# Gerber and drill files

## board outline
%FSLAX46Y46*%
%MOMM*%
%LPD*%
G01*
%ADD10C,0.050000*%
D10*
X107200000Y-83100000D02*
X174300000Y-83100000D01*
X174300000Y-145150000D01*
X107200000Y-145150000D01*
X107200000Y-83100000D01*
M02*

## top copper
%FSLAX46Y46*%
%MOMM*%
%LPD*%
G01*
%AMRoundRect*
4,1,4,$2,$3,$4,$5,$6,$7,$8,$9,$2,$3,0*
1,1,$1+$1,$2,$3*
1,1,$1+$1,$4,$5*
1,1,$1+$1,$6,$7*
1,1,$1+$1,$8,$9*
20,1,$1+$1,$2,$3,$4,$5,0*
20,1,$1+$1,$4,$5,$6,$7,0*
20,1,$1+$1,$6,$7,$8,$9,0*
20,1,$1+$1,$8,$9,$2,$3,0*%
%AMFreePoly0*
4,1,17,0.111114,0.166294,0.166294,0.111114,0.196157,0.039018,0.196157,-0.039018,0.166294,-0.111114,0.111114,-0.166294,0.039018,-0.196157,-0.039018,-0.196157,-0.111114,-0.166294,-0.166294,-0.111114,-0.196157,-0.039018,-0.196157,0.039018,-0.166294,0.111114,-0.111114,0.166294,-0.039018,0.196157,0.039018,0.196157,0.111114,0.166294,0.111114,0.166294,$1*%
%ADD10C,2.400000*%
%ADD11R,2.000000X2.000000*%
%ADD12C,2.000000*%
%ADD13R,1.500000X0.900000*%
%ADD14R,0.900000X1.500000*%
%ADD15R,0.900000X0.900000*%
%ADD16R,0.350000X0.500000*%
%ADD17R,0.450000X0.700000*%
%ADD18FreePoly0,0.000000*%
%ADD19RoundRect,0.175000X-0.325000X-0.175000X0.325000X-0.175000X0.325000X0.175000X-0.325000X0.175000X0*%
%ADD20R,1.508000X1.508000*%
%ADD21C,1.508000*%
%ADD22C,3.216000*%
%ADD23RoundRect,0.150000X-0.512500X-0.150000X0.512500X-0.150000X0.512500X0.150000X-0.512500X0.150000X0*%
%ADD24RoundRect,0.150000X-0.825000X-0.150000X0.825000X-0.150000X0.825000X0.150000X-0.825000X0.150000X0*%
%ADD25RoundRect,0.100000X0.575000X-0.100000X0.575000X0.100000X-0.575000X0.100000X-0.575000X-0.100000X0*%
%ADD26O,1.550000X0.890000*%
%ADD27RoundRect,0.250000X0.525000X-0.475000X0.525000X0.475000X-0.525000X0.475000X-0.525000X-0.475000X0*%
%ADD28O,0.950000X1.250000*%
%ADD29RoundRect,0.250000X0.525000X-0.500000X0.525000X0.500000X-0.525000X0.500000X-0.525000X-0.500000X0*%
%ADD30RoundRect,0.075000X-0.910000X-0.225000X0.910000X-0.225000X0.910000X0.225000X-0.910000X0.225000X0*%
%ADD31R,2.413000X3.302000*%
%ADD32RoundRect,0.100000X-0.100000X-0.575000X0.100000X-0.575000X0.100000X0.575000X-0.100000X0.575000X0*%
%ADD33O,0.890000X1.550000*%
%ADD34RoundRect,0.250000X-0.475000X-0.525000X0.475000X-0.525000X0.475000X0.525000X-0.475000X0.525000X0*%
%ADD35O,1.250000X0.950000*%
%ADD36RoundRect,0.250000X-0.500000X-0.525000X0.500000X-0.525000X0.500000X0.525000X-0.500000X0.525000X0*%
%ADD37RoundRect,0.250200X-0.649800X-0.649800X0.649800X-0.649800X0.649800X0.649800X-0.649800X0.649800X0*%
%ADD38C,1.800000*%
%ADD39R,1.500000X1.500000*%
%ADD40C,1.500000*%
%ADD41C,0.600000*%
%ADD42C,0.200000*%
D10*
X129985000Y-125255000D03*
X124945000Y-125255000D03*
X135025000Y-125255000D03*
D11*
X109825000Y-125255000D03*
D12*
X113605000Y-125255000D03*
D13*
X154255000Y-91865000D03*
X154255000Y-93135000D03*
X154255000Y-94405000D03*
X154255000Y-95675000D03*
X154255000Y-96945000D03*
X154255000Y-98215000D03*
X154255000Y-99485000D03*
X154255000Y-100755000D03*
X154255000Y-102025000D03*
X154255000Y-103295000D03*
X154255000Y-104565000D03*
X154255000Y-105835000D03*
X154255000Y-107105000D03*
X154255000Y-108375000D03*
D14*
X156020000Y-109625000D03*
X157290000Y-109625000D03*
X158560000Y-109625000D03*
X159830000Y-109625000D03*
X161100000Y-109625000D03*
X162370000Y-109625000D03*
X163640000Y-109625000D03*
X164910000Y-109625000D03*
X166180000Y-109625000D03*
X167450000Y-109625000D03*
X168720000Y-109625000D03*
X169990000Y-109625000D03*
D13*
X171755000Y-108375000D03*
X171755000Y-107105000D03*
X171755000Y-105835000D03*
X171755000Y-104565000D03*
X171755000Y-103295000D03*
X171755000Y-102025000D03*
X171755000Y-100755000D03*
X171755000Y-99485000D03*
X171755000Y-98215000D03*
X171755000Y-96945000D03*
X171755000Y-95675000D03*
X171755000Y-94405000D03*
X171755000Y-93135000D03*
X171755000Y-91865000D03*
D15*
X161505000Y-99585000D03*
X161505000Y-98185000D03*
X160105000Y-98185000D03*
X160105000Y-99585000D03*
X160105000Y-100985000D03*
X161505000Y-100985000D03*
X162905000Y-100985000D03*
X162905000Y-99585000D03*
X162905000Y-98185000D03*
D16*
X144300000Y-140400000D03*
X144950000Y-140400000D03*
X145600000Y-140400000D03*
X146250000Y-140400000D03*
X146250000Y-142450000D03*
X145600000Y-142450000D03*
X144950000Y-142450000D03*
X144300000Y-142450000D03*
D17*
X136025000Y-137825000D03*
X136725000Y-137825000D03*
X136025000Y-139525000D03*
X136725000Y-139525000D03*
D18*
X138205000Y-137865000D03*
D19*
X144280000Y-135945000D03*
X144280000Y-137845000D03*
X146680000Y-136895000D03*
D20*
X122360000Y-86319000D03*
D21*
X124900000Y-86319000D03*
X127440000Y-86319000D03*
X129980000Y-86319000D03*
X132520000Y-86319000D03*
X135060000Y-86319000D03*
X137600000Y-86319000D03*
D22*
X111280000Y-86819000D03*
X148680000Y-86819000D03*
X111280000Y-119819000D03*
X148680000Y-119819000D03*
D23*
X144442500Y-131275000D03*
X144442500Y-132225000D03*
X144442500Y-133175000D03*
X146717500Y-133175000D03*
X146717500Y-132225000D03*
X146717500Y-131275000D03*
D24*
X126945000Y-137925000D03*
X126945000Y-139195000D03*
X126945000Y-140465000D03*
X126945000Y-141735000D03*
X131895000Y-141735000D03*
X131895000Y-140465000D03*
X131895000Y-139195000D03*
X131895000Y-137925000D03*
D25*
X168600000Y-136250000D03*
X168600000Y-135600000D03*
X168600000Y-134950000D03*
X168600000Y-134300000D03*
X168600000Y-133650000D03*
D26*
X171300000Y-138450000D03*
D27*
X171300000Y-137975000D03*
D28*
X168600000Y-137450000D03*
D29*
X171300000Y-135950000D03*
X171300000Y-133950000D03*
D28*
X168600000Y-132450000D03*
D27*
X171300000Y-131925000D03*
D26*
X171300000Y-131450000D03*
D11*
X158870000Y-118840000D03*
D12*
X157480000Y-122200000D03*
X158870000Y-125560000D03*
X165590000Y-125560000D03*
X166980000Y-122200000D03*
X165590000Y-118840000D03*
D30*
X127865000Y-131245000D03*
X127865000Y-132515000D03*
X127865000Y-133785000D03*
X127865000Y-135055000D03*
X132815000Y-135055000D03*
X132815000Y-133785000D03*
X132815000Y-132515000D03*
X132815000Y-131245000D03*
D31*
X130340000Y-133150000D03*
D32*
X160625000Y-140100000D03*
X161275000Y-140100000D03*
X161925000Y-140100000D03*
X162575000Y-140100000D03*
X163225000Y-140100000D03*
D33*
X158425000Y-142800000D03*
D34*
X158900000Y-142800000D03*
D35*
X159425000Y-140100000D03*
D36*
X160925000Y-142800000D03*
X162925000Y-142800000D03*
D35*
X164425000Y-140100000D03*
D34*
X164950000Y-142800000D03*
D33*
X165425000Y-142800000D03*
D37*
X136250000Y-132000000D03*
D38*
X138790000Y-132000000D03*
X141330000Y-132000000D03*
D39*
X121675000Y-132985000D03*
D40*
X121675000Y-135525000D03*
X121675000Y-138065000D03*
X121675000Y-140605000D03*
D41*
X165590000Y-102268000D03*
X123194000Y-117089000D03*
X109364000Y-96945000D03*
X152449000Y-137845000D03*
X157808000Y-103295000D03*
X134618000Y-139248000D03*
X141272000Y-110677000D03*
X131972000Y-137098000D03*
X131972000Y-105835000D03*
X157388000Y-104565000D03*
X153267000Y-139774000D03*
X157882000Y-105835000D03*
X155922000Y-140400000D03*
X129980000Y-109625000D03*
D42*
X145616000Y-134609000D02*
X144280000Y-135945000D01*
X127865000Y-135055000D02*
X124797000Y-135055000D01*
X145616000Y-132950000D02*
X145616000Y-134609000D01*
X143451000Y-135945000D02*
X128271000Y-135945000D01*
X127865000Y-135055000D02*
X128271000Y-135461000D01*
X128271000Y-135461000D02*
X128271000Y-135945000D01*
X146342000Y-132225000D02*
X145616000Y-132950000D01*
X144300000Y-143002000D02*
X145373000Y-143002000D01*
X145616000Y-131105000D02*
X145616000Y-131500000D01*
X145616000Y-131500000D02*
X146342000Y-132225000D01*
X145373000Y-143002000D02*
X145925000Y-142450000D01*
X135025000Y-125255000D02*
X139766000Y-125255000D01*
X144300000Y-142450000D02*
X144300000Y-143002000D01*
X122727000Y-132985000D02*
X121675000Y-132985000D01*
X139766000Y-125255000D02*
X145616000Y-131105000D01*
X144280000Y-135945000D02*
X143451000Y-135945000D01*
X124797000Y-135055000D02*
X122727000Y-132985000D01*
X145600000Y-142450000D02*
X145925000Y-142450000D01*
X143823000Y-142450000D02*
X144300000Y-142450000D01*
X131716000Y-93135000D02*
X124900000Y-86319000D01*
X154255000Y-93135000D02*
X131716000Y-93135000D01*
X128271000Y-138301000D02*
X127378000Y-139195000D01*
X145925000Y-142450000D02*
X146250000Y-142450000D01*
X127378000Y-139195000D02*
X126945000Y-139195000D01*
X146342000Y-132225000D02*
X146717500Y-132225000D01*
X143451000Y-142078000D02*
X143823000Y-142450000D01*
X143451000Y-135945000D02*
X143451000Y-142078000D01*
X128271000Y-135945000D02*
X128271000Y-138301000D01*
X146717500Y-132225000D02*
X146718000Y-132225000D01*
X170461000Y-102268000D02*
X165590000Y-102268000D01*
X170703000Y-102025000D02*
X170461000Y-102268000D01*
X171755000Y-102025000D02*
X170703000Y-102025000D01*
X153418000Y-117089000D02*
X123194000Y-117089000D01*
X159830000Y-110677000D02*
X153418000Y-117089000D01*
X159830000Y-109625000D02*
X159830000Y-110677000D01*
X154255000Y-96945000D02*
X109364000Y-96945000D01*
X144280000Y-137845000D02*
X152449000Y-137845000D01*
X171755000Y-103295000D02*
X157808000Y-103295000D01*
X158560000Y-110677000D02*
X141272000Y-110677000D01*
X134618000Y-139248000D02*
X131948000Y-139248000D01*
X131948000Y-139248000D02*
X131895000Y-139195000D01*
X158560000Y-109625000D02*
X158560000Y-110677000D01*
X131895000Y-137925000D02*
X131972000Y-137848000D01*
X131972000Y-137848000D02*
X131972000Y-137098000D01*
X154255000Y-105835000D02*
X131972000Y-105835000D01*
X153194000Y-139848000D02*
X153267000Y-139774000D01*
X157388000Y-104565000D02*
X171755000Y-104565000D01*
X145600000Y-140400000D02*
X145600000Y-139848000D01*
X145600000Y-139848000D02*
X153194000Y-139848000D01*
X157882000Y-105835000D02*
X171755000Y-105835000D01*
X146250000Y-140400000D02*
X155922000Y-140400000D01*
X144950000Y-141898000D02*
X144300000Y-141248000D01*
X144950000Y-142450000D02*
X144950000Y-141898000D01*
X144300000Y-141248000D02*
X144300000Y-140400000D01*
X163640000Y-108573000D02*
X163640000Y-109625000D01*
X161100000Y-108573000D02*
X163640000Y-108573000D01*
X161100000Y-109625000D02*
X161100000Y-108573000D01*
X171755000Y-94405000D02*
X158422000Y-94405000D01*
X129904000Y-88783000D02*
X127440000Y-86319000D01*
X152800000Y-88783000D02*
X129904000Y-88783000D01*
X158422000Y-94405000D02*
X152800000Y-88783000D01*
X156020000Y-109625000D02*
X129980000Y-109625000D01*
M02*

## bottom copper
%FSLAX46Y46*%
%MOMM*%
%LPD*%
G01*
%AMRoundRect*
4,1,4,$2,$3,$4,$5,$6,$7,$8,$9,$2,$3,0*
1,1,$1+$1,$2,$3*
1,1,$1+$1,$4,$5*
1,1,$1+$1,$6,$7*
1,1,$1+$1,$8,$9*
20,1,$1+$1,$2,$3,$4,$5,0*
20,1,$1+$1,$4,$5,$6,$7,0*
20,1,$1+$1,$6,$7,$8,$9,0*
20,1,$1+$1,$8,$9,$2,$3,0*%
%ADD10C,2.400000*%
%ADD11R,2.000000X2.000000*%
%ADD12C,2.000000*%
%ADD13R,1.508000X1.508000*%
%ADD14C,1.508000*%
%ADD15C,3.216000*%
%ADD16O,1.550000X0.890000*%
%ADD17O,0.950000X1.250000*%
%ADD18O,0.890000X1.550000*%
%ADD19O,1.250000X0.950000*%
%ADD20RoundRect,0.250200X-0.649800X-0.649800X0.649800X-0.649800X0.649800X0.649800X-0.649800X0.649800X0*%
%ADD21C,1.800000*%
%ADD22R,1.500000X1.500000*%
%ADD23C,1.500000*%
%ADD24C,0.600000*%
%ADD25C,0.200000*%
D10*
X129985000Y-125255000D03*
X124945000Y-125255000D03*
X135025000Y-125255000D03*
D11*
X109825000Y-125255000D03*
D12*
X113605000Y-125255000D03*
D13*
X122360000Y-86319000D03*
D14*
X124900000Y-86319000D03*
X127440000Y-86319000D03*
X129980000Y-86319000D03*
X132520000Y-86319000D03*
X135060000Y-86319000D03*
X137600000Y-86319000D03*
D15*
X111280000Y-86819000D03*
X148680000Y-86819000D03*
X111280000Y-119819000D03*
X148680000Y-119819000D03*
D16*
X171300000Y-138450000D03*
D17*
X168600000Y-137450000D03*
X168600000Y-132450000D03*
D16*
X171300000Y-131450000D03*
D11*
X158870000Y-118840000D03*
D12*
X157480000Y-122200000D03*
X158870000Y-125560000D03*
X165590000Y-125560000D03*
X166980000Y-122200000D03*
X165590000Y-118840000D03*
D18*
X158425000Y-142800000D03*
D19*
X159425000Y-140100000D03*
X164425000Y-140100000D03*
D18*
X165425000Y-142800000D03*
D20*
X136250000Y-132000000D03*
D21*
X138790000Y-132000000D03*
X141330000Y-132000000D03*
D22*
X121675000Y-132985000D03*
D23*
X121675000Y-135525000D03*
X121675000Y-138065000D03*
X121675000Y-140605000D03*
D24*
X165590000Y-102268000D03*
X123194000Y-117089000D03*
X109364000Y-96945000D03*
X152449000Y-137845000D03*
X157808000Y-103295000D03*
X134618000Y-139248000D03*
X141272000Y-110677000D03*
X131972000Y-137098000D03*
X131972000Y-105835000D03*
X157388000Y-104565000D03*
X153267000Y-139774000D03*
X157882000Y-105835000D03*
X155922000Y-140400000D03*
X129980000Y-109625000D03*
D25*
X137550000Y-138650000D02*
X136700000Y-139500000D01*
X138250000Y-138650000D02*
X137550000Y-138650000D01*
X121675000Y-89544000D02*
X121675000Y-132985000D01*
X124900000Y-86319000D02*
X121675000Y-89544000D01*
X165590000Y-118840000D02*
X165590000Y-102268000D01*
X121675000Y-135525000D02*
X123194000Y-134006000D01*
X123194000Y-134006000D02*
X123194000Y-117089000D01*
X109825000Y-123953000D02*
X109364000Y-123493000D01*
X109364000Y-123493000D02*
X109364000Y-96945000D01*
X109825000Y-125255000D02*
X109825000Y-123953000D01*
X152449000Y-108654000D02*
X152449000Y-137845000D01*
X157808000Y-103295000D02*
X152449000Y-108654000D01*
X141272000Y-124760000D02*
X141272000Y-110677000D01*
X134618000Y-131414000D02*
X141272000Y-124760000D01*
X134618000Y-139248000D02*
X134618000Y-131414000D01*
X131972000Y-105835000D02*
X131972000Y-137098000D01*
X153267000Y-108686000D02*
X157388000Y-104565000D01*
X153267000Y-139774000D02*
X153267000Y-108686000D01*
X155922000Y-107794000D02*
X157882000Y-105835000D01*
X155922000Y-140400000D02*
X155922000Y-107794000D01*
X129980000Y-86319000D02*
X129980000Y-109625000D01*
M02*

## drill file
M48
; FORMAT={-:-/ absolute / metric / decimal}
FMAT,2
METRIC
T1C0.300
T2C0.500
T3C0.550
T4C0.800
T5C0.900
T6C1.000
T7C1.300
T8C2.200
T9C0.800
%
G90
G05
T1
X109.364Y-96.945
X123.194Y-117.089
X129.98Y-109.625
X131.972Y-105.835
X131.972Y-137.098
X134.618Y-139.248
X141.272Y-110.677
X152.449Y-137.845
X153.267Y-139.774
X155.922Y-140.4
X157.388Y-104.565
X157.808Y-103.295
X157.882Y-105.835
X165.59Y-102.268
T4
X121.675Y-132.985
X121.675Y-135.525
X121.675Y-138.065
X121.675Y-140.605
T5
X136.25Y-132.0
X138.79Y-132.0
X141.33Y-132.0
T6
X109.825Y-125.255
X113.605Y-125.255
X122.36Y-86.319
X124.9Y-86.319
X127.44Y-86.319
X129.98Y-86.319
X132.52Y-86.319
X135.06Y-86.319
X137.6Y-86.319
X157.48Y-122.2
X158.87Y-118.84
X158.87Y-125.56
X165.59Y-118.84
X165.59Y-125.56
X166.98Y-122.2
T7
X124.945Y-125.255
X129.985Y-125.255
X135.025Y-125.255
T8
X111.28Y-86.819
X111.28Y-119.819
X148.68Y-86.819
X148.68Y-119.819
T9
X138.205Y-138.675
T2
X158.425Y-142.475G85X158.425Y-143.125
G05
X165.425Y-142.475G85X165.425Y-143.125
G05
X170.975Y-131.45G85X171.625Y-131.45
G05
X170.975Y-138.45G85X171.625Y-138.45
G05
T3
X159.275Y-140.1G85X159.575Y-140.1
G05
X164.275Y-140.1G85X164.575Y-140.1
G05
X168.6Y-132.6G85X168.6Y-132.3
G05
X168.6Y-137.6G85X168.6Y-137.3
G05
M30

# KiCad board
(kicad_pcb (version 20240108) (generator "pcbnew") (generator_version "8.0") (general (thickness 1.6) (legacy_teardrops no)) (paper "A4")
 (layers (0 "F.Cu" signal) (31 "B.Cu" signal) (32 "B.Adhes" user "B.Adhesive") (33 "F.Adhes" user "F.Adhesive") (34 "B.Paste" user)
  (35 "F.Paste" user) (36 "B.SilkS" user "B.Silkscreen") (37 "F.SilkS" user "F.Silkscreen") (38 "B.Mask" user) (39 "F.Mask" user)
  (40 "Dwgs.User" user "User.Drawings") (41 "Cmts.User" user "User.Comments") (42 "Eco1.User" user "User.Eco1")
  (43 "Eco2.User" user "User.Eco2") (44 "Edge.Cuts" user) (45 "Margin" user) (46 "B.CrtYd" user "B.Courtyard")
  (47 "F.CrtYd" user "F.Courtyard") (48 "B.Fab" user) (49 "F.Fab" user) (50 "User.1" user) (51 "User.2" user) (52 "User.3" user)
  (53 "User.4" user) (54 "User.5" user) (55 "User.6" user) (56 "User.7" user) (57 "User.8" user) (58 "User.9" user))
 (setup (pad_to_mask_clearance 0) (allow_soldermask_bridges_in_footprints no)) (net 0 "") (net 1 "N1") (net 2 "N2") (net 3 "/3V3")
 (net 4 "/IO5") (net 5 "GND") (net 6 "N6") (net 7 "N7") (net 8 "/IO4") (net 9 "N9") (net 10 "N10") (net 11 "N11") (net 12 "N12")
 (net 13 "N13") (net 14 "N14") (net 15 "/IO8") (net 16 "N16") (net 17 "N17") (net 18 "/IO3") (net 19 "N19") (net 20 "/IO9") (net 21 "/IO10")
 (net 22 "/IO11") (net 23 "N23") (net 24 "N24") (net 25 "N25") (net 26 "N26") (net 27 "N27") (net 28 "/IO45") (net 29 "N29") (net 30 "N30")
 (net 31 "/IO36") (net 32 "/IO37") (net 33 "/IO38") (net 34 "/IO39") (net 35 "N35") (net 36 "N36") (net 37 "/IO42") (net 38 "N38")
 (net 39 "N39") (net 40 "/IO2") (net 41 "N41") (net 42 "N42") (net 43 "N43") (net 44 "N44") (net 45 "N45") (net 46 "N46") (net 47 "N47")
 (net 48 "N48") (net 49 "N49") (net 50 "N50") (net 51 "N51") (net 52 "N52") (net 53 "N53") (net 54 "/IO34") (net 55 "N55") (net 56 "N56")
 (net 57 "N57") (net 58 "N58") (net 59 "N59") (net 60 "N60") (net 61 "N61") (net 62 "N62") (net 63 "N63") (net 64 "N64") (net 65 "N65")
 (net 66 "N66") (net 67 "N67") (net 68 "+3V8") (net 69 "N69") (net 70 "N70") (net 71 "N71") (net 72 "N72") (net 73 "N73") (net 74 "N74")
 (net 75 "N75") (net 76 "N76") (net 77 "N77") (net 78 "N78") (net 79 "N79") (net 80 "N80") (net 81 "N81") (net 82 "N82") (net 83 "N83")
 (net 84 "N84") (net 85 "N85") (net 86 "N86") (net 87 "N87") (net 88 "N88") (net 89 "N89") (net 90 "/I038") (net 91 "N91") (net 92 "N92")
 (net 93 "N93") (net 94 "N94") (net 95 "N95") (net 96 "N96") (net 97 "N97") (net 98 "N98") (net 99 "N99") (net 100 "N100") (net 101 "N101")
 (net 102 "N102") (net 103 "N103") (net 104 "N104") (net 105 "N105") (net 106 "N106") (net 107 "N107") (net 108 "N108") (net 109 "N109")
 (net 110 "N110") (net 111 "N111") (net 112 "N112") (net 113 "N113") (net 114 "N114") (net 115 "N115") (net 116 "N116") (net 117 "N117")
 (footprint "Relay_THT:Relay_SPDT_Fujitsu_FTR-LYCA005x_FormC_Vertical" (layer "F.Cu") (at 109.825 125.255)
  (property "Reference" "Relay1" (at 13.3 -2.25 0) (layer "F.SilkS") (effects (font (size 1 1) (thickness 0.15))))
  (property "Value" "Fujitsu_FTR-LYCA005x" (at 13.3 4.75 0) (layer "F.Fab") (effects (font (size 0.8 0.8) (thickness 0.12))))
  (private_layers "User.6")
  (pad "11" thru_hole circle (at 20.16 0) (size 2.4 2.4) (drill 1.3) (layers "*.Cu" "*.Mask") (remove_unused_layers no) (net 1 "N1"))
  (pad "12" thru_hole circle (at 15.12 0) (size 2.4 2.4) (drill 1.3) (layers "*.Cu" "*.Mask") (remove_unused_layers no) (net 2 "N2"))
  (pad "14" thru_hole circle (at 25.2 0) (size 2.4 2.4) (drill 1.3) (layers "*.Cu" "*.Mask") (remove_unused_layers no) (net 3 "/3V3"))
  (pad "A1" thru_hole rect (at 0 0) (size 2 2) (drill 1) (layers "*.Cu" "*.Mask") (remove_unused_layers no) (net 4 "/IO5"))
  (pad "A2" thru_hole circle (at 3.78 0) (size 2 2) (drill 1) (layers "*.Cu" "*.Mask") (remove_unused_layers no) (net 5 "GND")))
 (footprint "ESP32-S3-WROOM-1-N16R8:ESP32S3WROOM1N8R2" (layer "F.Cu") (at 163.005 97.125)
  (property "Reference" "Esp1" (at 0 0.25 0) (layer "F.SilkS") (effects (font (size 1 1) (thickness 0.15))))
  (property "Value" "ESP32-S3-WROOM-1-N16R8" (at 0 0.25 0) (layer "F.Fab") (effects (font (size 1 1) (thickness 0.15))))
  (pad "1" smd rect (at -8.75 -5.26) (size 1.5 0.9) (layers "F.Cu" "F.Paste" "F.Mask") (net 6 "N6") (solder_mask_margin 0.102))
  (pad "2" smd rect (at -8.75 -3.99) (size 1.5 0.9) (layers "F.Cu" "F.Paste" "F.Mask") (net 3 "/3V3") (solder_mask_margin 0.102))
  (pad "3" smd rect (at -8.75 -2.72) (size 1.5 0.9) (layers "F.Cu" "F.Paste" "F.Mask") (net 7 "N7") (solder_mask_margin 0.102))
  (pad "4" smd rect (at -8.75 -1.45) (size 1.5 0.9) (layers "F.Cu" "F.Paste" "F.Mask") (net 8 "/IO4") (solder_mask_margin 0.102))
  (pad "5" smd rect (at -8.75 -0.18) (size 1.5 0.9) (layers "F.Cu" "F.Paste" "F.Mask") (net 4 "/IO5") (solder_mask_margin 0.102))
  (pad "6" smd rect (at -8.75 1.09) (size 1.5 0.9) (layers "F.Cu" "F.Paste" "F.Mask") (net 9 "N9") (solder_mask_margin 0.102))
  (pad "7" smd rect (at -8.75 2.36) (size 1.5 0.9) (layers "F.Cu" "F.Paste" "F.Mask") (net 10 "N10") (solder_mask_margin 0.102))
  (pad "8" smd rect (at -8.75 3.63) (size 1.5 0.9) (layers "F.Cu" "F.Paste" "F.Mask") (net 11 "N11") (solder_mask_margin 0.102))
  (pad "9" smd rect (at -8.75 4.9) (size 1.5 0.9) (layers "F.Cu" "F.Paste" "F.Mask") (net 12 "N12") (solder_mask_margin 0.102))
  (pad "10" smd rect (at -8.75 6.17) (size 1.5 0.9) (layers "F.Cu" "F.Paste" "F.Mask") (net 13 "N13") (solder_mask_margin 0.102))
  (pad "11" smd rect (at -8.75 7.44) (size 1.5 0.9) (layers "F.Cu" "F.Paste" "F.Mask") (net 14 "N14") (solder_mask_margin 0.102))
  (pad "12" smd rect (at -8.75 8.71) (size 1.5 0.9) (layers "F.Cu" "F.Paste" "F.Mask") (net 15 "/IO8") (solder_mask_margin 0.102))
  (pad "13" smd rect (at -8.75 9.98) (size 1.5 0.9) (layers "F.Cu" "F.Paste" "F.Mask") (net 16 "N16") (solder_mask_margin 0.102))
  (pad "14" smd rect (at -8.75 11.25) (size 1.5 0.9) (layers "F.Cu" "F.Paste" "F.Mask") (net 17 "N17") (solder_mask_margin 0.102))
  (pad "15" smd rect (at -6.985 12.5) (size 0.9 1.5) (layers "F.Cu" "F.Paste" "F.Mask") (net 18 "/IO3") (solder_mask_margin 0.102))
  (pad "16" smd rect (at -5.715 12.5) (size 0.9 1.5) (layers "F.Cu" "F.Paste" "F.Mask") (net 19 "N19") (solder_mask_margin 0.102))
  (pad "17" smd rect (at -4.445 12.5) (size 0.9 1.5) (layers "F.Cu" "F.Paste" "F.Mask") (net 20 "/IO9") (solder_mask_margin 0.102))
  (pad "18" smd rect (at -3.175 12.5) (size 0.9 1.5) (layers "F.Cu" "F.Paste" "F.Mask") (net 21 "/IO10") (solder_mask_margin 0.102))
  (pad "19" smd rect (at -1.905 12.5) (size 0.9 1.5) (layers "F.Cu" "F.Paste" "F.Mask") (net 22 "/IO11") (solder_mask_margin 0.102))
  (pad "20" smd rect (at -0.635 12.5) (size 0.9 1.5) (layers "F.Cu" "F.Paste" "F.Mask") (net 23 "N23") (solder_mask_margin 0.102))
  (pad "21" smd rect (at 0.635 12.5) (size 0.9 1.5) (layers "F.Cu" "F.Paste" "F.Mask") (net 22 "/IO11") (solder_mask_margin 0.102))
  (pad "22" smd rect (at 1.905 12.5) (size 0.9 1.5) (layers "F.Cu" "F.Paste" "F.Mask") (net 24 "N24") (solder_mask_margin 0.102))
  (pad "23" smd rect (at 3.175 12.5) (size 0.9 1.5) (layers "F.Cu" "F.Paste" "F.Mask") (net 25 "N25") (solder_mask_margin 0.102))
  (pad "24" smd rect (at 4.445 12.5) (size 0.9 1.5) (layers "F.Cu" "F.Paste" "F.Mask") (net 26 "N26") (solder_mask_margin 0.102))
  (pad "25" smd rect (at 5.715 12.5) (size 0.9 1.5) (layers "F.Cu" "F.Paste" "F.Mask") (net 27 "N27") (solder_mask_margin 0.102))
  (pad "26" smd rect (at 6.985 12.5) (size 0.9 1.5) (layers "F.Cu" "F.Paste" "F.Mask") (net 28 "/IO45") (solder_mask_margin 0.102))
  (pad "27" smd rect (at 8.75 11.25) (size 1.5 0.9) (layers "F.Cu" "F.Paste" "F.Mask") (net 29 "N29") (solder_mask_margin 0.102))
  (pad "28" smd rect (at 8.75 9.98) (size 1.5 0.9) (layers "F.Cu" "F.Paste" "F.Mask") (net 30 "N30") (solder_mask_margin 0.102))
  (pad "29" smd rect (at 8.75 8.71) (size 1.5 0.9) (layers "F.Cu" "F.Paste" "F.Mask") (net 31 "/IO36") (solder_mask_margin 0.102))
  (pad "30" smd rect (at 8.75 7.44) (size 1.5 0.9) (layers "F.Cu" "F.Paste" "F.Mask") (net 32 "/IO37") (solder_mask_margin 0.102))
  (pad "31" smd rect (at 8.75 6.17) (size 1.5 0.9) (layers "F.Cu" "F.Paste" "F.Mask") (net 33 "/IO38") (solder_mask_margin 0.102))
  (pad "32" smd rect (at 8.75 4.9) (size 1.5 0.9) (layers "F.Cu" "F.Paste" "F.Mask") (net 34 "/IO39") (solder_mask_margin 0.102))
  (pad "33" smd rect (at 8.75 3.63) (size 1.5 0.9) (layers "F.Cu" "F.Paste" "F.Mask") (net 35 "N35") (solder_mask_margin 0.102))
  (pad "34" smd rect (at 8.75 2.36) (size 1.5 0.9) (layers "F.Cu" "F.Paste" "F.Mask") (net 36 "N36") (solder_mask_margin 0.102))
  (pad "35" smd rect (at 8.75 1.09) (size 1.5 0.9) (layers "F.Cu" "F.Paste" "F.Mask") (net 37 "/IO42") (solder_mask_margin 0.102))
  (pad "36" smd rect (at 8.75 -0.18) (size 1.5 0.9) (layers "F.Cu" "F.Paste" "F.Mask") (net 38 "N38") (solder_mask_margin 0.102))
  (pad "37" smd rect (at 8.75 -1.45) (size 1.5 0.9) (layers "F.Cu" "F.Paste" "F.Mask") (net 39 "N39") (solder_mask_margin 0.102))
  (pad "38" smd rect (at 8.75 -2.72) (size 1.5 0.9) (layers "F.Cu" "F.Paste" "F.Mask") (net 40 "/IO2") (solder_mask_margin 0.102))
  (pad "39" smd rect (at 8.75 -3.99) (size 1.5 0.9) (layers "F.Cu" "F.Paste" "F.Mask") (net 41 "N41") (solder_mask_margin 0.102))
  (pad "40" smd rect (at 8.75 -5.26) (size 1.5 0.9) (layers "F.Cu" "F.Paste" "F.Mask") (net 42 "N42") (solder_mask_margin 0.102))
  (pad "41" smd rect (at -1.5 2.46) (size 0.9 0.9) (layers "F.Cu" "F.Paste" "F.Mask") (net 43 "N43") (solder_mask_margin 0.102))
  (pad "42" smd rect (at -1.5 1.06) (size 0.9 0.9) (layers "F.Cu" "F.Paste" "F.Mask") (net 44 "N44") (solder_mask_margin 0.102))
  (pad "43" smd rect (at -2.9 1.06) (size 0.9 0.9) (layers "F.Cu" "F.Paste" "F.Mask") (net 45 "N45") (solder_mask_margin 0.102))
  (pad "44" smd rect (at -2.9 2.46) (size 0.9 0.9) (layers "F.Cu" "F.Paste" "F.Mask") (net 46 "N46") (solder_mask_margin 0.102))
  (pad "45" smd rect (at -2.9 3.86) (size 0.9 0.9) (layers "F.Cu" "F.Paste" "F.Mask") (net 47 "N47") (solder_mask_margin 0.102))
  (pad "46" smd rect (at -1.5 3.86) (size 0.9 0.9) (layers "F.Cu" "F.Paste" "F.Mask") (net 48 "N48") (solder_mask_margin 0.102))
  (pad "47" smd rect (at -0.1 3.86) (size 0.9 0.9) (layers "F.Cu" "F.Paste" "F.Mask") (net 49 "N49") (solder_mask_margin 0.102))
  (pad "48" smd rect (at -0.1 2.46) (size 0.9 0.9) (layers "F.Cu" "F.Paste" "F.Mask") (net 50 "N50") (solder_mask_margin 0.102))
  (pad "49" smd rect (at -0.1 1.06) (size 0.9 0.9) (layers "F.Cu" "F.Paste" "F.Mask") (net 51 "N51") (solder_mask_margin 0.102)))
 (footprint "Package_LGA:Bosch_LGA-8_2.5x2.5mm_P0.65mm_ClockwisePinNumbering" (layer "F.Cu") (at 145.275 141.425)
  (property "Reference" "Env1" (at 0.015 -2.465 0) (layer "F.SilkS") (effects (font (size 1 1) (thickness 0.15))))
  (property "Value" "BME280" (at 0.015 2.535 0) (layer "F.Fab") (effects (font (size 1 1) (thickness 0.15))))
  (pad "1" smd rect (at -0.975 -1.025 90) (size 0.5 0.35) (layers "F.Cu" "F.Paste" "F.Mask") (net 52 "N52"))
  (pad "2" smd rect (at -0.325 -1.025 90) (size 0.5 0.35) (layers "F.Cu" "F.Paste" "F.Mask") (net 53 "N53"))
  (pad "3" smd rect (at 0.325 -1.025 90) (size 0.5 0.35) (layers "F.Cu" "F.Paste" "F.Mask") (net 32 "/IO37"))
  (pad "4" smd rect (at 0.975 -1.025 90) (size 0.5 0.35) (layers "F.Cu" "F.Paste" "F.Mask") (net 31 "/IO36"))
  (pad "5" smd rect (at 0.975 1.025 90) (size 0.5 0.35) (layers "F.Cu" "F.Paste" "F.Mask") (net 3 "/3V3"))
  (pad "6" smd rect (at 0.325 1.025 90) (size 0.5 0.35) (layers "F.Cu" "F.Paste" "F.Mask") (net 3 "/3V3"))
  (pad "7" smd rect (at -0.325 1.025 90) (size 0.5 0.35) (layers "F.Cu" "F.Paste" "F.Mask") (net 52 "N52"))
  (pad "8" smd rect (at -0.975 1.025 90) (size 0.5 0.35) (layers "F.Cu" "F.Paste" "F.Mask") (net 3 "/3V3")))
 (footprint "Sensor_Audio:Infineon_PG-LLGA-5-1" (layer "F.Cu") (at 137.525 138.675)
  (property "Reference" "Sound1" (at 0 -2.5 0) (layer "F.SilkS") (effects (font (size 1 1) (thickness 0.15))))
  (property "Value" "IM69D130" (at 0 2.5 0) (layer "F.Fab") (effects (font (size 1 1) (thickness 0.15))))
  (pad "" smd custom (at -1.5 -0.725) (size 0.3 0.3) (layers "F.Paste") (zone_connect 0) (options (clearance outline) (anchor circle))
   (primitives))
  (pad "" smd custom (at -1.5 0.725) (size 0.3 0.3) (layers "F.Paste") (zone_connect 0) (options (clearance outline) (anchor circle))
   (primitives))
  (pad "" smd custom (at -0.8 -0.725) (size 0.3 0.3) (layers "F.Paste") (zone_connect 0) (options (clearance outline) (anchor circle))
   (primitives))
  (pad "" smd custom (at -0.8 0.725) (size 0.3 0.3) (layers "F.Paste") (zone_connect 0) (options (clearance outline) (anchor circle))
   (primitives))
  (pad "" smd custom (at -0.12 0) (size 0.3 0.3) (layers "F.Paste") (zone_connect 0) (options (clearance outline) (anchor circle))
   (primitives))
  (pad "" smd custom (at 0.28 -0.693) (size 0.3 0.3) (layers "F.Paste") (zone_connect 0) (options (clearance outline) (anchor circle))
   (primitives))
  (pad "" smd custom (at 0.28 0.693) (size 0.3 0.3) (layers "F.Paste") (zone_connect 0) (options (clearance outline) (anchor circle))
   (primitives))
  (pad "" np_thru_hole circle (at 0.68 0) (size 0.8 0.8) (drill 0.8) (layers "*.Cu" "*.Mask"))
  (pad "" smd custom (at 1.08 -0.693) (size 0.3 0.3) (layers "F.Paste") (zone_connect 0) (options (clearance outline) (anchor circle))
   (primitives))
  (pad "" smd custom (at 1.08 0.693) (size 0.3 0.3) (layers "F.Paste") (zone_connect 0) (options (clearance outline) (anchor circle))
   (primitives))
  (pad "" smd custom (at 1.48 0) (size 0.3 0.3) (layers "F.Paste") (zone_connect 0) (options (clearance outline) (anchor circle))
   (primitives))
  (pad "1" smd rect (at -1.5 -0.85) (size 0.45 0.7) (layers "F.Cu" "F.Mask") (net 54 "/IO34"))
  (pad "2" smd rect (at -0.8 -0.85) (size 0.45 0.7) (layers "F.Cu" "F.Mask") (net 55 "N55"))
  (pad "3" smd rect (at -1.5 0.85) (size 0.45 0.7) (layers "F.Cu" "F.Mask") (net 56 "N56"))
  (pad "4" smd rect (at -0.8 0.85) (size 0.45 0.7) (layers "F.Cu" "F.Mask") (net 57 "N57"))
  (pad "5" smd custom (at 0.68 -0.81) (size 0.4 0.4) (layers "F.Cu" "F.Mask") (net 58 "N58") (zone_connect 0)
   (options (clearance outline) (anchor circle)) (primitives)))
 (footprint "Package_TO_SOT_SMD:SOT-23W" (layer "F.Cu") (at 145.48 136.895)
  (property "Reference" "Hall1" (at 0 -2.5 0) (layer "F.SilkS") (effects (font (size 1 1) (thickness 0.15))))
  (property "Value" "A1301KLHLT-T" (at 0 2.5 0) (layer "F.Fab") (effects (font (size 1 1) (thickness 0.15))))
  (pad "1" smd roundrect (at -1.2 -0.95) (size 1 0.7) (layers "F.Cu" "F.Paste" "F.Mask") (roundrect_rratio 0.25) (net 3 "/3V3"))
  (pad "2" smd roundrect (at -1.2 0.95) (size 1 0.7) (layers "F.Cu" "F.Paste" "F.Mask") (roundrect_rratio 0.25) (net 33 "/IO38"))
  (pad "3" smd roundrect (at 1.2 0) (size 1 0.7) (layers "F.Cu" "F.Paste" "F.Mask") (roundrect_rratio 0.25) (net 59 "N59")))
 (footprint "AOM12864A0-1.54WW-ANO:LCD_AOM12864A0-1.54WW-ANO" (layer "F.Cu") (at 129.98 103.319)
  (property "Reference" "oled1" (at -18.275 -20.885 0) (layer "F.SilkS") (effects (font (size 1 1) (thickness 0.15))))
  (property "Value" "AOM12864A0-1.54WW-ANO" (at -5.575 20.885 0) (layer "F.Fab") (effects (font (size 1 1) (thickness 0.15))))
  (pad "1" thru_hole rect (at -7.62 -17) (size 1.508 1.508) (drill 1) (layers "*.Cu" "*.Mask") (remove_unused_layers no) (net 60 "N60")
   (solder_mask_margin 0.102))
  (pad "2" thru_hole circle (at -5.08 -17) (size 1.508 1.508) (drill 1) (layers "*.Cu" "*.Mask") (remove_unused_layers no) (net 3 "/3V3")
   (solder_mask_margin 0.102))
  (pad "3" thru_hole circle (at -2.54 -17) (size 1.508 1.508) (drill 1) (layers "*.Cu" "*.Mask") (remove_unused_layers no) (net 40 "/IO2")
   (solder_mask_margin 0.102))
  (pad "4" thru_hole circle (at 0 -17) (size 1.508 1.508) (drill 1) (layers "*.Cu" "*.Mask") (remove_unused_layers no) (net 18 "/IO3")
   (solder_mask_margin 0.102))
  (pad "5" thru_hole circle (at 2.54 -17) (size 1.508 1.508) (drill 1) (layers "*.Cu" "*.Mask") (remove_unused_layers no) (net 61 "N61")
   (solder_mask_margin 0.102))
  (pad "6" thru_hole circle (at 5.08 -17) (size 1.508 1.508) (drill 1) (layers "*.Cu" "*.Mask") (remove_unused_layers no) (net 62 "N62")
   (solder_mask_margin 0.102))
  (pad "7" thru_hole circle (at 7.62 -17) (size 1.508 1.508) (drill 1) (layers "*.Cu" "*.Mask") (remove_unused_layers no) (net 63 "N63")
   (solder_mask_margin 0.102))
  (pad "P1" thru_hole circle (at -18.7 -16.5) (size 3.216 3.216) (drill 2.2) (layers "*.Cu" "*.Mask") (remove_unused_layers no)
   (solder_mask_margin 0.102))
  (pad "P2" thru_hole circle (at 18.7 -16.5) (size 3.216 3.216) (drill 2.2) (layers "*.Cu" "*.Mask") (remove_unused_layers no)
   (solder_mask_margin 0.102))
  (pad "P3" thru_hole circle (at -18.7 16.5) (size 3.216 3.216) (drill 2.2) (layers "*.Cu" "*.Mask") (remove_unused_layers no)
   (solder_mask_margin 0.102))
  (pad "P4" thru_hole circle (at 18.7 16.5) (size 3.216 3.216) (drill 2.2) (layers "*.Cu" "*.Mask") (remove_unused_layers no)
   (solder_mask_margin 0.102)))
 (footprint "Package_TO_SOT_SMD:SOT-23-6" (layer "F.Cu") (at 145.58 132.225)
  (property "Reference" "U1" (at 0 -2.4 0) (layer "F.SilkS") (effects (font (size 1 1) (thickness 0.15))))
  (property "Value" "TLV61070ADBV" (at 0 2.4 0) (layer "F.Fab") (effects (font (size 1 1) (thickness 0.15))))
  (pad "1" smd roundrect (at -1.1375 -0.95) (size 1.325 0.6) (layers "F.Cu" "F.Paste" "F.Mask") (roundrect_rratio 0.25) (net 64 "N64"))
  (pad "2" smd roundrect (at -1.1375 0) (size 1.325 0.6) (layers "F.Cu" "F.Paste" "F.Mask") (roundrect_rratio 0.25) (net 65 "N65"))
  (pad "3" smd roundrect (at -1.1375 0.95) (size 1.325 0.6) (layers "F.Cu" "F.Paste" "F.Mask") (roundrect_rratio 0.25) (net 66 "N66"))
  (pad "4" smd roundrect (at 1.1375 0.95) (size 1.325 0.6) (layers "F.Cu" "F.Paste" "F.Mask") (roundrect_rratio 0.25) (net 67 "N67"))
  (pad "5" smd roundrect (at 1.1375 0) (size 1.325 0.6) (layers "F.Cu" "F.Paste" "F.Mask") (roundrect_rratio 0.25) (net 3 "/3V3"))
  (pad "6" smd roundrect (at 1.1375 -0.95) (size 1.325 0.6) (layers "F.Cu" "F.Paste" "F.Mask") (roundrect_rratio 0.25) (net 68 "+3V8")))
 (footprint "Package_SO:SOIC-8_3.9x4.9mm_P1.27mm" (layer "F.Cu") (at 129.42 139.83)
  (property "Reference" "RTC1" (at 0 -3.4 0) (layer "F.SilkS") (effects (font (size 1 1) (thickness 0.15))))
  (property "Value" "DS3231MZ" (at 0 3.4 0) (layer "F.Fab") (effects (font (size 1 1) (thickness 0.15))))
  (pad "1" smd roundrect (at -2.475 -1.905) (size 1.95 0.6) (layers "F.Cu" "F.Paste" "F.Mask") (roundrect_rratio 0.25) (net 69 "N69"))
  (pad "2" smd roundrect (at -2.475 -0.635) (size 1.95 0.6) (layers "F.Cu" "F.Paste" "F.Mask") (roundrect_rratio 0.25) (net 3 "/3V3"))
  (pad "3" smd roundrect (at -2.475 0.635) (size 1.95 0.6) (layers "F.Cu" "F.Paste" "F.Mask") (roundrect_rratio 0.25) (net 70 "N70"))
  (pad "4" smd roundrect (at -2.475 1.905) (size 1.95 0.6) (layers "F.Cu" "F.Paste" "F.Mask") (roundrect_rratio 0.25) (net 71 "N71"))
  (pad "5" smd roundrect (at 2.475 1.905) (size 1.95 0.6) (layers "F.Cu" "F.Paste" "F.Mask") (roundrect_rratio 0.25) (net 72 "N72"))
  (pad "6" smd roundrect (at 2.475 0.635) (size 1.95 0.6) (layers "F.Cu" "F.Paste" "F.Mask") (roundrect_rratio 0.25) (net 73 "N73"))
  (pad "7" smd roundrect (at 2.475 -0.635) (size 1.95 0.6) (layers "F.Cu" "F.Paste" "F.Mask") (roundrect_rratio 0.25) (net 20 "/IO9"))
  (pad "8" smd roundrect (at 2.475 -1.905) (size 1.95 0.6) (layers "F.Cu" "F.Paste" "F.Mask") (roundrect_rratio 0.25) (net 15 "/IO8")))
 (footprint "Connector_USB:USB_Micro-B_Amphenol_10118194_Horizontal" (layer "F.Cu") (at 170 134.95 90)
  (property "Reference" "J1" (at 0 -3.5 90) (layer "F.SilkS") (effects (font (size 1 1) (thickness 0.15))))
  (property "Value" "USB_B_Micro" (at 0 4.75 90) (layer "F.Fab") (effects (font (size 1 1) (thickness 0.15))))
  (pad "" smd oval (at -3.5 1.3 90) (size 0.89 1.55) (layers "F.Paste"))
  (pad "" smd oval (at -2.5 -1.4 90) (size 1.25 0.95) (layers "F.Paste"))
  (pad "" smd oval (at 2.5 -1.4 90) (size 1.25 0.95) (layers "F.Paste"))
  (pad "" smd oval (at 3.5 1.3 90) (size 0.89 1.55) (layers "F.Paste"))
  (pad "1" smd roundrect (at -1.3 -1.4 90) (size 0.4 1.35) (layers "F.Cu" "F.Paste" "F.Mask") (roundrect_rratio 0.25) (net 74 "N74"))
  (pad "2" smd roundrect (at -0.65 -1.4 90) (size 0.4 1.35) (layers "F.Cu" "F.Paste" "F.Mask") (roundrect_rratio 0.25) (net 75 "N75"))
  (pad "3" smd roundrect (at 0 -1.4 90) (size 0.4 1.35) (layers "F.Cu" "F.Paste" "F.Mask") (roundrect_rratio 0.25) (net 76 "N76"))
  (pad "4" smd roundrect (at 0.65 -1.4 90) (size 0.4 1.35) (layers "F.Cu" "F.Paste" "F.Mask") (roundrect_rratio 0.25) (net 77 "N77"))
  (pad "5" smd roundrect (at 1.3 -1.4 90) (size 0.4 1.35) (layers "F.Cu" "F.Paste" "F.Mask") (roundrect_rratio 0.25) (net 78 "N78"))
  (pad "6" thru_hole oval (at -3.5 1.3 90) (size 0.89 1.55) (drill oval 0.5 1.15) (layers "*.Cu" "*.Mask") (remove_unused_layers no)
   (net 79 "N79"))
  (pad "6" smd roundrect (at -3.025 1.3 90) (size 1.45 1.55) (layers "F.Cu" "F.Paste" "F.Mask") (roundrect_rratio 0.1724137931)
   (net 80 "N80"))
  (pad "6" thru_hole oval (at -2.5 -1.4 90) (size 1.25 0.95) (drill oval 0.85 0.55) (layers "*.Cu" "*.Mask") (remove_unused_layers no)
   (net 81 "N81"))
  (pad "6" smd roundrect (at -1 1.3 90) (size 1.5 1.55) (layers "F.Cu" "F.Paste" "F.Mask") (roundrect_rratio 0.1666666667) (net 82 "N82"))
  (pad "6" smd roundrect (at 1 1.3 90) (size 1.5 1.55) (layers "F.Cu" "F.Paste" "F.Mask") (roundrect_rratio 0.1666666667) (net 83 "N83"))
  (pad "6" thru_hole oval (at 2.5 -1.4 90) (size 1.25 0.95) (drill oval 0.85 0.55) (layers "*.Cu" "*.Mask") (remove_unused_layers no)
   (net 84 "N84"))
  (pad "6" smd roundrect (at 3.025 1.3 90) (size 1.45 1.55) (layers "F.Cu" "F.Paste" "F.Mask") (roundrect_rratio 0.1724137931)
   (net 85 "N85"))
  (pad "6" thru_hole oval (at 3.5 1.3 90) (size 0.89 1.55) (drill oval 0.5 1.15) (layers "*.Cu" "*.Mask") (remove_unused_layers no)
   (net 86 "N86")))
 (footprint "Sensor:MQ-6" (layer "F.Cu") (at 158.87 118.84)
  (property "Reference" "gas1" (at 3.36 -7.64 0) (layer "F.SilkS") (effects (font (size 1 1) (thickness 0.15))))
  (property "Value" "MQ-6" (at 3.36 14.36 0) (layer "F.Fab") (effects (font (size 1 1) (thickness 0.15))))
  (pad "1" thru_hole rect (at 0 0) (size 2 2) (drill 1) (layers "*.Cu" "*.Mask") (remove_unused_layers no) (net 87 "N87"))
  (pad "2" thru_hole circle (at -1.39 3.36) (size 2 2) (drill 1) (layers "*.Cu" "*.Mask") (remove_unused_layers no) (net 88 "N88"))
  (pad "3" thru_hole circle (at 0 6.72 90) (size 2 2) (drill 1) (layers "*.Cu" "*.Mask") (remove_unused_layers no) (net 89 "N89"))
  (pad "4" thru_hole circle (at 6.72 6.72 180) (size 2 2) (drill 1) (layers "*.Cu" "*.Mask") (remove_unused_layers no) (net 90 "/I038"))
  (pad "5" thru_hole circle (at 8.11 3.36) (size 2 2) (drill 1) (layers "*.Cu" "*.Mask") (remove_unused_layers no) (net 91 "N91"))
  (pad "6" thru_hole circle (at 6.72 0 270) (size 2 2) (drill 1) (layers "*.Cu" "*.Mask") (remove_unused_layers no) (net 34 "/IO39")))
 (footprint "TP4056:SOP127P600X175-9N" (layer "F.Cu") (at 130.34 133.15)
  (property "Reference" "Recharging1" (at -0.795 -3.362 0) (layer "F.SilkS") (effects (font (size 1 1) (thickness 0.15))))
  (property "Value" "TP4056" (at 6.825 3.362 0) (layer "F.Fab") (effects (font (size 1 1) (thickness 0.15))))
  (pad "1" smd roundrect (at -2.475 -1.905) (size 1.97 0.6) (layers "F.Cu" "F.Paste" "F.Mask") (roundrect_rratio 0.125) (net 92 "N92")
   (solder_mask_margin 0.102))
  (pad "2" smd roundrect (at -2.475 -0.635) (size 1.97 0.6) (layers "F.Cu" "F.Paste" "F.Mask") (roundrect_rratio 0.125) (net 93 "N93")
   (solder_mask_margin 0.102))
  (pad "3" smd roundrect (at -2.475 0.635) (size 1.97 0.6) (layers "F.Cu" "F.Paste" "F.Mask") (roundrect_rratio 0.125) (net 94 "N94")
   (solder_mask_margin 0.102))
  (pad "4" smd roundrect (at -2.475 1.905) (size 1.97 0.6) (layers "F.Cu" "F.Paste" "F.Mask") (roundrect_rratio 0.125) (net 3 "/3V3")
   (solder_mask_margin 0.102))
  (pad "5" smd roundrect (at 2.475 1.905) (size 1.97 0.6) (layers "F.Cu" "F.Paste" "F.Mask") (roundrect_rratio 0.125) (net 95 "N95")
   (solder_mask_margin 0.102))
  (pad "6" smd roundrect (at 2.475 0.635) (size 1.97 0.6) (layers "F.Cu" "F.Paste" "F.Mask") (roundrect_rratio 0.125) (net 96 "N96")
   (solder_mask_margin 0.102))
  (pad "7" smd roundrect (at 2.475 -0.635) (size 1.97 0.6) (layers "F.Cu" "F.Paste" "F.Mask") (roundrect_rratio 0.125) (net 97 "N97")
   (solder_mask_margin 0.102))
  (pad "8" smd roundrect (at 2.475 -1.905) (size 1.97 0.6) (layers "F.Cu" "F.Paste" "F.Mask") (roundrect_rratio 0.125) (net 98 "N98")
   (solder_mask_margin 0.102))
  (pad "9" smd rect (at 0 0) (size 2.413 3.302) (layers "F.Cu" "F.Mask") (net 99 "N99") (solder_mask_margin 0.102)))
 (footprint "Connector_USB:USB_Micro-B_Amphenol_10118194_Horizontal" (layer "F.Cu") (at 161.925 141.5)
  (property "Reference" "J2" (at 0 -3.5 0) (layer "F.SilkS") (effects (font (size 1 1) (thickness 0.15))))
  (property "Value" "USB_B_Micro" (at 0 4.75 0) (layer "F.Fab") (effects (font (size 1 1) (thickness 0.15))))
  (pad "" smd oval (at -3.5 1.3) (size 0.89 1.55) (layers "F.Paste"))
  (pad "" smd oval (at -2.5 -1.4) (size 1.25 0.95) (layers "F.Paste"))
  (pad "" smd oval (at 2.5 -1.4) (size 1.25 0.95) (layers "F.Paste"))
  (pad "" smd oval (at 3.5 1.3) (size 0.89 1.55) (layers "F.Paste"))
  (pad "1" smd roundrect (at -1.3 -1.4) (size 0.4 1.35) (layers "F.Cu" "F.Paste" "F.Mask") (roundrect_rratio 0.25) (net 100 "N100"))
  (pad "2" smd roundrect (at -0.65 -1.4) (size 0.4 1.35) (layers "F.Cu" "F.Paste" "F.Mask") (roundrect_rratio 0.25) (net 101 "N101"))
  (pad "3" smd roundrect (at 0 -1.4) (size 0.4 1.35) (layers "F.Cu" "F.Paste" "F.Mask") (roundrect_rratio 0.25) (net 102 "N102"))
  (pad "4" smd roundrect (at 0.65 -1.4) (size 0.4 1.35) (layers "F.Cu" "F.Paste" "F.Mask") (roundrect_rratio 0.25) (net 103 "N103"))
  (pad "5" smd roundrect (at 1.3 -1.4) (size 0.4 1.35) (layers "F.Cu" "F.Paste" "F.Mask") (roundrect_rratio 0.25) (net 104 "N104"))
  (pad "6" thru_hole oval (at -3.5 1.3) (size 0.89 1.55) (drill oval 0.5 1.15) (layers "*.Cu" "*.Mask") (remove_unused_layers no)
   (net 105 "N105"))
  (pad "6" smd roundrect (at -3.025 1.3) (size 1.45 1.55) (layers "F.Cu" "F.Paste" "F.Mask") (roundrect_rratio 0.1724137931)
   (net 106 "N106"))
  (pad "6" thru_hole oval (at -2.5 -1.4) (size 1.25 0.95) (drill oval 0.85 0.55) (layers "*.Cu" "*.Mask") (remove_unused_layers no)
   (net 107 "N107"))
  (pad "6" smd roundrect (at -1 1.3) (size 1.5 1.55) (layers "F.Cu" "F.Paste" "F.Mask") (roundrect_rratio 0.1666666667) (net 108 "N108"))
  (pad "6" smd roundrect (at 1 1.3) (size 1.5 1.55) (layers "F.Cu" "F.Paste" "F.Mask") (roundrect_rratio 0.1666666667) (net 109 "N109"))
  (pad "6" thru_hole oval (at 2.5 -1.4) (size 1.25 0.95) (drill oval 0.85 0.55) (layers "*.Cu" "*.Mask") (remove_unused_layers no)
   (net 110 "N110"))
  (pad "6" smd roundrect (at 3.025 1.3) (size 1.45 1.55) (layers "F.Cu" "F.Paste" "F.Mask") (roundrect_rratio 0.1724137931) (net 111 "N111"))
  (pad "6" thru_hole oval (at 3.5 1.3) (size 0.89 1.55) (drill oval 0.5 1.15) (layers "*.Cu" "*.Mask") (remove_unused_layers no)
   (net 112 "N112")))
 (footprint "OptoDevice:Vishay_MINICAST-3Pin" (layer "F.Cu") (at 136.25 132)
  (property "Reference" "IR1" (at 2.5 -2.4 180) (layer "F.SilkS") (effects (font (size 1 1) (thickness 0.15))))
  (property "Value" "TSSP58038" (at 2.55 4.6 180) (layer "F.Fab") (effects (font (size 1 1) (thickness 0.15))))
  (pad "1" thru_hole roundrect (at 0 0) (size 1.8 1.8) (drill 0.9) (layers "*.Cu" "*.Mask") (remove_unused_layers no)
   (roundrect_rratio 0.139) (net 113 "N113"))
  (pad "2" thru_hole circle (at 2.54 0) (size 1.8 1.8) (drill 0.9) (layers "*.Cu" "*.Mask") (remove_unused_layers no) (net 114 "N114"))
  (pad "3" thru_hole circle (at 5.08 0) (size 1.8 1.8) (drill 0.9) (layers "*.Cu" "*.Mask") (remove_unused_layers no) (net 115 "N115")))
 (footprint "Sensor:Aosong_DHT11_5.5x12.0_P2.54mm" (layer "F.Cu") (at 121.675 132.985)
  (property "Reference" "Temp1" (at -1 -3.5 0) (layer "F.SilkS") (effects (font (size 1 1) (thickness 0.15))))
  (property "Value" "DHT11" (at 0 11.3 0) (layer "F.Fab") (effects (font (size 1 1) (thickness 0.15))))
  (pad "1" thru_hole rect (at 0 0) (size 1.5 1.5) (drill 0.8) (layers "*.Cu" "*.Mask") (remove_unused_layers no) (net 3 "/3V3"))
  (pad "2" thru_hole circle (at 0 2.54) (size 1.5 1.5) (drill 0.8) (layers "*.Cu" "*.Mask") (remove_unused_layers no) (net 21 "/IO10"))
  (pad "3" thru_hole circle (at 0 5.08) (size 1.5 1.5) (drill 0.8) (layers "*.Cu" "*.Mask") (remove_unused_layers no) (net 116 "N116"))
  (pad "4" thru_hole circle (at 0 7.62) (size 1.5 1.5) (drill 0.8) (layers "*.Cu" "*.Mask") (remove_unused_layers no) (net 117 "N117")))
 (gr_rect (start 107.2 83.1) (end 174.3 145.15) (stroke (width 0.05) (type default)) (fill none) (layer "Edge.Cuts"))
 (segment (start 137.55 138.65) (end 136.7 139.5) (width 0.2) (layer "B.Cu") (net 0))
 (segment (start 138.25 138.65) (end 137.55 138.65) (width 0.2) (layer "B.Cu") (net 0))
 (segment (start 145.616 134.609) (end 144.28 135.945) (width 0.2) (layer "F.Cu") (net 3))
 (segment (start 127.865 135.055) (end 124.797 135.055) (width 0.2) (layer "F.Cu") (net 3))
 (segment (start 145.616 132.95) (end 145.616 134.609) (width 0.2) (layer "F.Cu") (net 3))
 (segment (start 143.451 135.945) (end 128.271 135.945) (width 0.2) (layer "F.Cu") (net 3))
 (segment (start 127.865 135.055) (end 128.271 135.461) (width 0.2) (layer "F.Cu") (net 3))
 (segment (start 128.271 135.461) (end 128.271 135.945) (width 0.2) (layer "F.Cu") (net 3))
 (segment (start 146.342 132.225) (end 145.616 132.95) (width 0.2) (layer "F.Cu") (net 3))
 (segment (start 144.3 143.002) (end 145.373 143.002) (width 0.2) (layer "F.Cu") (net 3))
 (segment (start 145.616 131.105) (end 145.616 131.5) (width 0.2) (layer "F.Cu") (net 3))
 (segment (start 145.616 131.5) (end 146.342 132.225) (width 0.2) (layer "F.Cu") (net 3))
 (segment (start 145.373 143.002) (end 145.925 142.45) (width 0.2) (layer "F.Cu") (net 3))
 (segment (start 135.025 125.255) (end 139.766 125.255) (width 0.2) (layer "F.Cu") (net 3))
 (segment (start 144.3 142.45) (end 144.3 143.002) (width 0.2) (layer "F.Cu") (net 3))
 (segment (start 122.727 132.985) (end 121.675 132.985) (width 0.2) (layer "F.Cu") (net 3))
 (segment (start 139.766 125.255) (end 145.616 131.105) (width 0.2) (layer "F.Cu") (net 3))
 (segment (start 144.28 135.945) (end 143.451 135.945) (width 0.2) (layer "F.Cu") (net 3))
 (segment (start 124.797 135.055) (end 122.727 132.985) (width 0.2) (layer "F.Cu") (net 3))
 (segment (start 145.6 142.45) (end 145.925 142.45) (width 0.2) (layer "F.Cu") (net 3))
 (segment (start 143.823 142.45) (end 144.3 142.45) (width 0.2) (layer "F.Cu") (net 3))
 (segment (start 131.716 93.135) (end 124.9 86.319) (width 0.2) (layer "F.Cu") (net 3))
 (segment (start 154.255 93.135) (end 131.716 93.135) (width 0.2) (layer "F.Cu") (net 3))
 (segment (start 128.271 138.301) (end 127.378 139.195) (width 0.2) (layer "F.Cu") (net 3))
 (segment (start 145.925 142.45) (end 146.25 142.45) (width 0.2) (layer "F.Cu") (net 3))
 (segment (start 127.378 139.195) (end 126.945 139.195) (width 0.2) (layer "F.Cu") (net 3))
 (segment (start 146.342 132.225) (end 146.7175 132.225) (width 0.2) (layer "F.Cu") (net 3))
 (segment (start 143.451 142.078) (end 143.823 142.45) (width 0.2) (layer "F.Cu") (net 3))
 (segment (start 143.451 135.945) (end 143.451 142.078) (width 0.2) (layer "F.Cu") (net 3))
 (segment (start 128.271 135.945) (end 128.271 138.301) (width 0.2) (layer "F.Cu") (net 3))
 (segment (start 146.7175 132.225) (end 146.718 132.225) (width 0.2) (layer "F.Cu") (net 3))
 (segment (start 121.675 89.544) (end 121.675 132.985) (width 0.2) (layer "B.Cu") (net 3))
 (segment (start 124.9 86.319) (end 121.675 89.544) (width 0.2) (layer "B.Cu") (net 3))
 (segment (start 170.461 102.268) (end 165.59 102.268) (width 0.2) (layer "F.Cu") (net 34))
 (segment (start 170.703 102.025) (end 170.461 102.268) (width 0.2) (layer "F.Cu") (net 34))
 (segment (start 171.755 102.025) (end 170.703 102.025) (width 0.2) (layer "F.Cu") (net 34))
 (via (at 165.59 102.268) (size 0.6) (drill 0.3) (layers "F.Cu" "B.Cu") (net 34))
 (segment (start 165.59 118.84) (end 165.59 102.268) (width 0.2) (layer "B.Cu") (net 34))
 (segment (start 153.418 117.089) (end 123.194 117.089) (width 0.2) (layer "F.Cu") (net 21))
 (segment (start 159.83 110.677) (end 153.418 117.089) (width 0.2) (layer "F.Cu") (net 21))
 (segment (start 159.83 109.625) (end 159.83 110.677) (width 0.2) (layer "F.Cu") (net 21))
 (via (at 123.194 117.089) (size 0.6) (drill 0.3) (layers "F.Cu" "B.Cu") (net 21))
 (segment (start 121.675 135.525) (end 123.194 134.006) (width 0.2) (layer "B.Cu") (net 21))
 (segment (start 123.194 134.006) (end 123.194 117.089) (width 0.2) (layer "B.Cu") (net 21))
 (segment (start 154.255 96.945) (end 109.364 96.945) (width 0.2) (layer "F.Cu") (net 4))
 (via (at 109.364 96.945) (size 0.6) (drill 0.3) (layers "F.Cu" "B.Cu") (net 4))
 (segment (start 109.825 123.953) (end 109.364 123.493) (width 0.2) (layer "B.Cu") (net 4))
 (segment (start 109.364 123.493) (end 109.364 96.945) (width 0.2) (layer "B.Cu") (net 4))
 (segment (start 109.825 125.255) (end 109.825 123.953) (width 0.2) (layer "B.Cu") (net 4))
 (segment (start 144.28 137.845) (end 152.449 137.845) (width 0.2) (layer "F.Cu") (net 33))
 (segment (start 171.755 103.295) (end 157.808 103.295) (width 0.2) (layer "F.Cu") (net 33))
 (via (at 152.449 137.845) (size 0.6) (drill 0.3) (layers "F.Cu" "B.Cu") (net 33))
 (via (at 157.808 103.295) (size 0.6) (drill 0.3) (layers "F.Cu" "B.Cu") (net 33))
 (segment (start 152.449 108.654) (end 152.449 137.845) (width 0.2) (layer "B.Cu") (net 33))
 (segment (start 157.808 103.295) (end 152.449 108.654) (width 0.2) (layer "B.Cu") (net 33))
 (segment (start 158.56 110.677) (end 141.272 110.677) (width 0.2) (layer "F.Cu") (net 20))
 (segment (start 134.618 139.248) (end 131.948 139.248) (width 0.2) (layer "F.Cu") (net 20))
 (segment (start 131.948 139.248) (end 131.895 139.195) (width 0.2) (layer "F.Cu") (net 20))
 (segment (start 158.56 109.625) (end 158.56 110.677) (width 0.2) (layer "F.Cu") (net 20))
 (via (at 134.618 139.248) (size 0.6) (drill 0.3) (layers "F.Cu" "B.Cu") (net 20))
 (via (at 141.272 110.677) (size 0.6) (drill 0.3) (layers "F.Cu" "B.Cu") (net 20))
 (segment (start 141.272 124.76) (end 141.272 110.677) (width 0.2) (layer "B.Cu") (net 20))
 (segment (start 134.618 131.414) (end 141.272 124.76) (width 0.2) (layer "B.Cu") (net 20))
 (segment (start 134.618 139.248) (end 134.618 131.414) (width 0.2) (layer "B.Cu") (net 20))
 (segment (start 131.895 137.925) (end 131.972 137.848) (width 0.2) (layer "F.Cu") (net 15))
 (segment (start 131.972 137.848) (end 131.972 137.098) (width 0.2) (layer "F.Cu") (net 15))
 (segment (start 154.255 105.835) (end 131.972 105.835) (width 0.2) (layer "F.Cu") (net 15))
 (via (at 131.972 137.098) (size 0.6) (drill 0.3) (layers "F.Cu" "B.Cu") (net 15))
 (via (at 131.972 105.835) (size 0.6) (drill 0.3) (layers "F.Cu" "B.Cu") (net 15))
 (segment (start 131.972 105.835) (end 131.972 137.098) (width 0.2) (layer "B.Cu") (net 15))
 (segment (start 153.194 139.848) (end 153.267 139.774) (width 0.2) (layer "F.Cu") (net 32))
 (segment (start 157.388 104.565) (end 171.755 104.565) (width 0.2) (layer "F.Cu") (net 32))
 (segment (start 145.6 140.4) (end 145.6 139.848) (width 0.2) (layer "F.Cu") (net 32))
 (segment (start 145.6 139.848) (end 153.194 139.848) (width 0.2) (layer "F.Cu") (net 32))
 (via (at 157.388 104.565) (size 0.6) (drill 0.3) (layers "F.Cu" "B.Cu") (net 32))
 (via (at 153.267 139.774) (size 0.6) (drill 0.3) (layers "F.Cu" "B.Cu") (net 32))
 (segment (start 153.267 108.686) (end 157.388 104.565) (width 0.2) (layer "B.Cu") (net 32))
 (segment (start 153.267 139.774) (end 153.267 108.686) (width 0.2) (layer "B.Cu") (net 32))
 (segment (start 157.882 105.835) (end 171.755 105.835) (width 0.2) (layer "F.Cu") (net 31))
 (segment (start 146.25 140.4) (end 155.922 140.4) (width 0.2) (layer "F.Cu") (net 31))
 (via (at 157.882 105.835) (size 0.6) (drill 0.3) (layers "F.Cu" "B.Cu") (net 31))
 (via (at 155.922 140.4) (size 0.6) (drill 0.3) (layers "F.Cu" "B.Cu") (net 31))
 (segment (start 155.922 107.794) (end 157.882 105.835) (width 0.2) (layer "B.Cu") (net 31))
 (segment (start 155.922 140.4) (end 155.922 107.794) (width 0.2) (layer "B.Cu") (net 31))
 (segment (start 144.95 141.898) (end 144.3 141.248) (width 0.2) (layer "F.Cu") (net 52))
 (segment (start 144.95 142.45) (end 144.95 141.898) (width 0.2) (layer "F.Cu") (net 52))
 (segment (start 144.3 141.248) (end 144.3 140.4) (width 0.2) (layer "F.Cu") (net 52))
 (segment (start 163.64 108.573) (end 163.64 109.625) (width 0.2) (layer "F.Cu") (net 22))
 (segment (start 161.1 108.573) (end 163.64 108.573) (width 0.2) (layer "F.Cu") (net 22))
 (segment (start 161.1 109.625) (end 161.1 108.573) (width 0.2) (layer "F.Cu") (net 22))
 (segment (start 171.755 94.405) (end 158.422 94.405) (width 0.2) (layer "F.Cu") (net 40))
 (segment (start 129.904 88.783) (end 127.44 86.319) (width 0.2) (layer "F.Cu") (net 40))
 (segment (start 152.8 88.783) (end 129.904 88.783) (width 0.2) (layer "F.Cu") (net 40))
 (segment (start 158.422 94.405) (end 152.8 88.783) (width 0.2) (layer "F.Cu") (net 40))
 (segment (start 156.02 109.625) (end 129.98 109.625) (width 0.2) (layer "F.Cu") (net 18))
 (via (at 129.98 109.625) (size 0.6) (drill 0.3) (layers "F.Cu" "B.Cu") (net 18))
 (segment (start 129.98 86.319) (end 129.98 109.625) (width 0.2) (layer "B.Cu") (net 18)))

